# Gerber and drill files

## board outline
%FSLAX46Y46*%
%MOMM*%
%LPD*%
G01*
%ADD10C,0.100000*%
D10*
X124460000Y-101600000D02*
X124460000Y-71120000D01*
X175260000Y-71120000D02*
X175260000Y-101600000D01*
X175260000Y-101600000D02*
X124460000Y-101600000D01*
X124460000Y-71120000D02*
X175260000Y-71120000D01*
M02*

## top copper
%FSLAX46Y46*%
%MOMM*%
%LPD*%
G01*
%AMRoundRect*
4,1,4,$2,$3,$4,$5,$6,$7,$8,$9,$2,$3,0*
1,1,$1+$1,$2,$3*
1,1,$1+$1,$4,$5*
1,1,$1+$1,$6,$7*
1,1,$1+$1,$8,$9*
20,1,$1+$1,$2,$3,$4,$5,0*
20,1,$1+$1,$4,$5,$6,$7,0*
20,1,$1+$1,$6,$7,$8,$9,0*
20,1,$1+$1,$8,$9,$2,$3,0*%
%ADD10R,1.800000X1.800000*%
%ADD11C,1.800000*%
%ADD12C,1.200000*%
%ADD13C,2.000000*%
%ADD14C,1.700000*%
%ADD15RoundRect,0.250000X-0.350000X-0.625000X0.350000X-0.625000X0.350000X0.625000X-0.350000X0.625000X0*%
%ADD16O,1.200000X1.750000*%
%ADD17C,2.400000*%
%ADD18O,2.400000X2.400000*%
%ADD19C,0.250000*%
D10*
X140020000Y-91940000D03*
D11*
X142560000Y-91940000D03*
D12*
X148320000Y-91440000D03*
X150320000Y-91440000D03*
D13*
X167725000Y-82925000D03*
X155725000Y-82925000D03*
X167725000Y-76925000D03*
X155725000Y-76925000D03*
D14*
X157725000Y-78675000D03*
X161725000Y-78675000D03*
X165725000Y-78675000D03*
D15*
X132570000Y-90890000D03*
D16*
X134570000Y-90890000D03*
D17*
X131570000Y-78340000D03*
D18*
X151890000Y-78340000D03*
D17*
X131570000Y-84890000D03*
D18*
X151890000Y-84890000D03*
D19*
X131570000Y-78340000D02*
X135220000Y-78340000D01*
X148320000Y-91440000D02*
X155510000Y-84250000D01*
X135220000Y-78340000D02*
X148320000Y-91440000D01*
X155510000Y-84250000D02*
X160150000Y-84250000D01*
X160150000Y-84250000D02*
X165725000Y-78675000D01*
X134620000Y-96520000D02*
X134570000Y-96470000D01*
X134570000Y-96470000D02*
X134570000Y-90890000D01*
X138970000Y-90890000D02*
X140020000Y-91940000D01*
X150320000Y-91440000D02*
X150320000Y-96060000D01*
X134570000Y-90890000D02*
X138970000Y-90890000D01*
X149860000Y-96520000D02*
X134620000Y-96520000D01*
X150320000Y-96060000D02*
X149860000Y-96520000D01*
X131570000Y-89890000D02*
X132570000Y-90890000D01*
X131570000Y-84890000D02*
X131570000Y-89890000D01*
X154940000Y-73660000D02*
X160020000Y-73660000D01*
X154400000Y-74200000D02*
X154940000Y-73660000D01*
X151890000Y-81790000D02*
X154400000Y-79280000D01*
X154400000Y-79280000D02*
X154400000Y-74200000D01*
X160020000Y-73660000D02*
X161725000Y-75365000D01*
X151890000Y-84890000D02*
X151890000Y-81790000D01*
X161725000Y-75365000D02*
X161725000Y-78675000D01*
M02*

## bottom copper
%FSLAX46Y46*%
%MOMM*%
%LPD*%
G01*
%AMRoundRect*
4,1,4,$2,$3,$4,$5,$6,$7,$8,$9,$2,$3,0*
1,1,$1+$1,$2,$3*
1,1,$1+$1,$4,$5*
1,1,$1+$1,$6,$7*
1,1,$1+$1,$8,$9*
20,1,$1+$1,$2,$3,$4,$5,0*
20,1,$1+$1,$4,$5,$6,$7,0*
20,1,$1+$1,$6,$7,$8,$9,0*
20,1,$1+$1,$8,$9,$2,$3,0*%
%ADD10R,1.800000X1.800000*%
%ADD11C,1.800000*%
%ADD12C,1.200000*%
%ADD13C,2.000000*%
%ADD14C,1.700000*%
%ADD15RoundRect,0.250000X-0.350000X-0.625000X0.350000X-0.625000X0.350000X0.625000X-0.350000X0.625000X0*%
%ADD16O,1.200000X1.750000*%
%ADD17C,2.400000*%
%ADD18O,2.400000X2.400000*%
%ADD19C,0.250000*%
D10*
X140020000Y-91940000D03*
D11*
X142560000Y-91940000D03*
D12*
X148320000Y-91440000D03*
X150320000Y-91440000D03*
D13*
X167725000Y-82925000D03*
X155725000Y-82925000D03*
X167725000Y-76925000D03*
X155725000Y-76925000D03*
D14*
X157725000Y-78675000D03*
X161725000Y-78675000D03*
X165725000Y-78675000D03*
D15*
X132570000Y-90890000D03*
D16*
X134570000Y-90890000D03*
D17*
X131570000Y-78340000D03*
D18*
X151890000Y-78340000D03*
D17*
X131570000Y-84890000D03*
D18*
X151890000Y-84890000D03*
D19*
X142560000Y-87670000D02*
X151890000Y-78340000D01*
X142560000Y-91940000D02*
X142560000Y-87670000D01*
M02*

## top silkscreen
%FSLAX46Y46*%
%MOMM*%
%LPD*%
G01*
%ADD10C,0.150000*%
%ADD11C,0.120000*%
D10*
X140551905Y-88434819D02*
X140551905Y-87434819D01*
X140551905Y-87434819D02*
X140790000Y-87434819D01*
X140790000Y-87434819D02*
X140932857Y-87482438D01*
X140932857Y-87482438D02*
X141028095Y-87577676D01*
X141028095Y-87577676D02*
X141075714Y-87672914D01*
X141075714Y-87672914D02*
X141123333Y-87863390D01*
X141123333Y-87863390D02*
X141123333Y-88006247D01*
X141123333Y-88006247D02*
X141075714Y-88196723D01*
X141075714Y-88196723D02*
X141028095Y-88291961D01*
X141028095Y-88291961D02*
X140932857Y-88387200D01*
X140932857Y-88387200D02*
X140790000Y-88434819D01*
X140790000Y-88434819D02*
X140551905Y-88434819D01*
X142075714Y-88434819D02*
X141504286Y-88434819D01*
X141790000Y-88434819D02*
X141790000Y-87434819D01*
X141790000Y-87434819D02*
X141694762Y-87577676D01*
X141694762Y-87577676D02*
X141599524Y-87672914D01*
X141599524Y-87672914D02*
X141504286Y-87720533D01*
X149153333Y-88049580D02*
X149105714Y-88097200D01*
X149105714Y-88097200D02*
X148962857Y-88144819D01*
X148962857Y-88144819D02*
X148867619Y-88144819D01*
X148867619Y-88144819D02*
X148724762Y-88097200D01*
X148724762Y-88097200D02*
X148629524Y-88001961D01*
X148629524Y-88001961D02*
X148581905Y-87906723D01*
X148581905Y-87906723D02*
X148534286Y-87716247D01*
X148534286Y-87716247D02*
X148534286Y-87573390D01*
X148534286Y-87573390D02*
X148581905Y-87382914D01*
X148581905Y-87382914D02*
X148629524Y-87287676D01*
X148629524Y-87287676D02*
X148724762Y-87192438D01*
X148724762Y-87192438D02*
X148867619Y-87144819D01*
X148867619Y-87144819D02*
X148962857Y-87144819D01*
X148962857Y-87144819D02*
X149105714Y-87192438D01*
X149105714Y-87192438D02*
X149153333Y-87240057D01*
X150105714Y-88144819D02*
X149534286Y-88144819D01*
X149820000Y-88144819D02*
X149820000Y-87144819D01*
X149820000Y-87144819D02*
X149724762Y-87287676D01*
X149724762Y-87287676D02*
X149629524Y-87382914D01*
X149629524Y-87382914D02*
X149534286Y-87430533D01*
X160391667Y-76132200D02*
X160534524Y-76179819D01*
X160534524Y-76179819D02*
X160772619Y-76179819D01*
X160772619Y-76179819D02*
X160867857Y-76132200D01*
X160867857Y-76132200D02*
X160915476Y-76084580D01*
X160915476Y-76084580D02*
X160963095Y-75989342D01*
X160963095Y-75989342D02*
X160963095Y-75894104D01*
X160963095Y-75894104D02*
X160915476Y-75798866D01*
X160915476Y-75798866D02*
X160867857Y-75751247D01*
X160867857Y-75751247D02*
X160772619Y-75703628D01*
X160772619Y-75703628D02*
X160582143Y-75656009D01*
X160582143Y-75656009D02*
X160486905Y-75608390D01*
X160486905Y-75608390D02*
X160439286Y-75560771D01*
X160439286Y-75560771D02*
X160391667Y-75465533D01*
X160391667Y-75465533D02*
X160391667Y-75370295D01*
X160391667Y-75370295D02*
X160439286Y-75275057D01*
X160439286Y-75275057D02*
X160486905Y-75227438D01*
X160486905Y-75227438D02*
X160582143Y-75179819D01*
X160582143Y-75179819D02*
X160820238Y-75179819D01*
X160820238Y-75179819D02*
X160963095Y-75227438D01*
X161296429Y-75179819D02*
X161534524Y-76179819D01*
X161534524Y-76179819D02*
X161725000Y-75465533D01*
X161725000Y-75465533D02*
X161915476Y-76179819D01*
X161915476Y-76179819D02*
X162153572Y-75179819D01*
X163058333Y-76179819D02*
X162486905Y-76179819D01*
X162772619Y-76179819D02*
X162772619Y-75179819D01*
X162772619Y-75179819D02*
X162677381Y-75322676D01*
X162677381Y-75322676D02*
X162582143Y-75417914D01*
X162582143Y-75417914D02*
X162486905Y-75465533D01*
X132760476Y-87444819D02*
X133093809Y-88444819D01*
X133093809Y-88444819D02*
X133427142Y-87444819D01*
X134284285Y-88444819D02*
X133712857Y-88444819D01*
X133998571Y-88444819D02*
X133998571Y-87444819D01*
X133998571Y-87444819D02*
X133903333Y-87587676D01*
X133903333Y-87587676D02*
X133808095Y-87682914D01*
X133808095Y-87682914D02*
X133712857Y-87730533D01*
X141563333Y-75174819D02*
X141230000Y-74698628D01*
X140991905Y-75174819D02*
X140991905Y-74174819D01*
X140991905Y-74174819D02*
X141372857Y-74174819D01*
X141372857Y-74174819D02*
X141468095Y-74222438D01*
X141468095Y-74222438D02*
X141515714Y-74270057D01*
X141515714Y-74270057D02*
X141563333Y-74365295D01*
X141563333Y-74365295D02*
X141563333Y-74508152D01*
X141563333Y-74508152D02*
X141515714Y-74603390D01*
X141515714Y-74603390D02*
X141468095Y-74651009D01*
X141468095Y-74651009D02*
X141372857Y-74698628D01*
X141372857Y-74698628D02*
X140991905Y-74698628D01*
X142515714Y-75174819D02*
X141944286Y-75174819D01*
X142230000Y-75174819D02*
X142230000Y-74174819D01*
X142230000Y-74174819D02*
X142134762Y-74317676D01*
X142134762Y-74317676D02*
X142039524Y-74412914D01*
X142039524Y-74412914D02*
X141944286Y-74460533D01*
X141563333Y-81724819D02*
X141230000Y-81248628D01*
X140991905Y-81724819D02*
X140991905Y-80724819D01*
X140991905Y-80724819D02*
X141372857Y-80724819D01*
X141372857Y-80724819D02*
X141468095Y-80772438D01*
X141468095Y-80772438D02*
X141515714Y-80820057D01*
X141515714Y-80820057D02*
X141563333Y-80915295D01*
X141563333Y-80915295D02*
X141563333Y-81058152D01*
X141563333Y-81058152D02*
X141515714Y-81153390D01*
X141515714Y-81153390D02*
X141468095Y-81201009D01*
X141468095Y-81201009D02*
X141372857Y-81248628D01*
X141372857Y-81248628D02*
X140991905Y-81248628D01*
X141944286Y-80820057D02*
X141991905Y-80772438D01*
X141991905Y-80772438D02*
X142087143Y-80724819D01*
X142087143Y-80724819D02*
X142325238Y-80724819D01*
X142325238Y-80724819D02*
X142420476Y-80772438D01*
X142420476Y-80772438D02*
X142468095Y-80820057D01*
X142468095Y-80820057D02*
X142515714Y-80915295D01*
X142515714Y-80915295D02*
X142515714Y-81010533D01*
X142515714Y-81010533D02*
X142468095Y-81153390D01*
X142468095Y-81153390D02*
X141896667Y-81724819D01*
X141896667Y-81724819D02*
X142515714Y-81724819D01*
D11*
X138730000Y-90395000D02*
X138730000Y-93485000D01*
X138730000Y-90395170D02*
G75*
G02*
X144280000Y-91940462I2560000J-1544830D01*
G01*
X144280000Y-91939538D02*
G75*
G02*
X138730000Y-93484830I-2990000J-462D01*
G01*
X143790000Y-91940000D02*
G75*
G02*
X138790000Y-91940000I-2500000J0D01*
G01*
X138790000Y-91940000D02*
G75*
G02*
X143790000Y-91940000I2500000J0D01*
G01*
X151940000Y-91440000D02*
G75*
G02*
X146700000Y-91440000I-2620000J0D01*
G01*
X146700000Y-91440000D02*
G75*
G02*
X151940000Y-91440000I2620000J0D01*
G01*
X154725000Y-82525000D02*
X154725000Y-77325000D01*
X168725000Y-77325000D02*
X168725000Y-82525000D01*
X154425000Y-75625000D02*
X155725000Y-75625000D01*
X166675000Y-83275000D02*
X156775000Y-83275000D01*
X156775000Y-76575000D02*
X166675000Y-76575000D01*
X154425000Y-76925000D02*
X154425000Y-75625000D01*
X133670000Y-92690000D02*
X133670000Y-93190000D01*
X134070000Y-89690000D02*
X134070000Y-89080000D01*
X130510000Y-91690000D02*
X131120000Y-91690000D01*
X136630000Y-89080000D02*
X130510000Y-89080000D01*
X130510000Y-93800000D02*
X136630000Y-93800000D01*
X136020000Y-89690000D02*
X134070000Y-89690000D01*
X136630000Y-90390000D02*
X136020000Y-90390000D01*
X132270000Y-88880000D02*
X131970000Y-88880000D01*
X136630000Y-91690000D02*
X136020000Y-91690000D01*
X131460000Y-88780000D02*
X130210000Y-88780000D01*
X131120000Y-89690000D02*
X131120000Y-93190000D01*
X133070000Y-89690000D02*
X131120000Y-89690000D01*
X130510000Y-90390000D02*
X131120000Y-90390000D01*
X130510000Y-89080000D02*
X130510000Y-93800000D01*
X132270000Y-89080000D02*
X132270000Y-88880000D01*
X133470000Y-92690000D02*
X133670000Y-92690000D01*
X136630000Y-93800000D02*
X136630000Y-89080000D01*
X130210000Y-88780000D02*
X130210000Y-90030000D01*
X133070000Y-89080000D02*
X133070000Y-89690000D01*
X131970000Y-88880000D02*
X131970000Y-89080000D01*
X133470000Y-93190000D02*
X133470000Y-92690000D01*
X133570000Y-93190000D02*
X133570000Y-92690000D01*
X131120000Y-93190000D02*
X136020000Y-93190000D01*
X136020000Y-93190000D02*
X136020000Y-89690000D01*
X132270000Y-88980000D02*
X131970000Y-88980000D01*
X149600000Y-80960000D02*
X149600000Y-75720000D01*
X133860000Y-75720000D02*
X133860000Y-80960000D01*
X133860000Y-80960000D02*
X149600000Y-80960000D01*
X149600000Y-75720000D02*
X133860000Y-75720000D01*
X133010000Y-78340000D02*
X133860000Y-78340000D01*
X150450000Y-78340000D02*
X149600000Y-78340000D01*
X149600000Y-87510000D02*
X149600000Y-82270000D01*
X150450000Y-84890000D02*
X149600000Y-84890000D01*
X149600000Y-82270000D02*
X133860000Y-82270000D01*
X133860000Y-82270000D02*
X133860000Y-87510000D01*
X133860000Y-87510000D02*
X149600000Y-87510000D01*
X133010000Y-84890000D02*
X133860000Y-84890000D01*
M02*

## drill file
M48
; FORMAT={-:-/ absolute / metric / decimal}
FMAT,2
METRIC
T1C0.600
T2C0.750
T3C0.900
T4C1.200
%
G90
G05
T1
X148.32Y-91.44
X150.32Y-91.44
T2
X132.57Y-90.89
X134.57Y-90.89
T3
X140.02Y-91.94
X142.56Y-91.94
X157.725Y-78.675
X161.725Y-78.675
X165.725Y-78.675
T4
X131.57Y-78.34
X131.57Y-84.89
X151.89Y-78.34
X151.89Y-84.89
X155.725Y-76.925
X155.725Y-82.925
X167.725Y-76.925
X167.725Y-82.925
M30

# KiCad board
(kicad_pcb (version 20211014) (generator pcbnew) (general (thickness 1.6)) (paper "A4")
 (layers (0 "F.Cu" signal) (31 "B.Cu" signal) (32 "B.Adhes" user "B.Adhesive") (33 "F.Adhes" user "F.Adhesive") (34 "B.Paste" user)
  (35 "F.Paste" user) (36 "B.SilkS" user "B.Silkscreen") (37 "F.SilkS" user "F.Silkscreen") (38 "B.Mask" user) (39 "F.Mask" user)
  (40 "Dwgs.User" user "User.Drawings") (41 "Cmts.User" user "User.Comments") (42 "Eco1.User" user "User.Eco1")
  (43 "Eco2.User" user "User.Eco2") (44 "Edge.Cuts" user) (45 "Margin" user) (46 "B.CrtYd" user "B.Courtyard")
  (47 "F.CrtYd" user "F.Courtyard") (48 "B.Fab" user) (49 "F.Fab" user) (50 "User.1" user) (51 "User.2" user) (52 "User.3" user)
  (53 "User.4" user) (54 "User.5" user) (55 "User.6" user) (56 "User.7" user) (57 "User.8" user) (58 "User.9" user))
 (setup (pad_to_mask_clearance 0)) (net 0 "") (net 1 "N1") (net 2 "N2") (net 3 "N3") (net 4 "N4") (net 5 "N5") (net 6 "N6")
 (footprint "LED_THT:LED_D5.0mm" (layer "F.Cu") (at 140.02 91.94)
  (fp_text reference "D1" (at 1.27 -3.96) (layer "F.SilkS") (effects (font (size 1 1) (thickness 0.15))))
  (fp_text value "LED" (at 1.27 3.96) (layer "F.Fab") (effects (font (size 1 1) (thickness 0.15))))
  (fp_line (start -1.29 -1.545) (end -1.29 1.545) (layer "F.SilkS") (width 0.12))
  (fp_arc (start -1.29 -1.54483) (mid 2.072002 -2.880433) (end 4.26 0.000462) (layer "F.SilkS") (width 0.12))
  (fp_arc (start 4.26 -0.000462) (mid 2.072002 2.880433) (end -1.29 1.54483) (layer "F.SilkS") (width 0.12))
  (fp_circle (center 1.27 0) (end 3.77 0) (layer "F.SilkS") (width 0.12) (fill none))
  (pad "1" thru_hole rect (at 0 0) (size 1.8 1.8) (drill 0.9) (layers *.Cu *.Mask) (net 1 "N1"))
  (pad "2" thru_hole circle (at 2.54 0) (size 1.8 1.8) (drill 0.9) (layers *.Cu *.Mask) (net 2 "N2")))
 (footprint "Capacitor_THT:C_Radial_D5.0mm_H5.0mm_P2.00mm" (layer "F.Cu") (at 148.32 91.44)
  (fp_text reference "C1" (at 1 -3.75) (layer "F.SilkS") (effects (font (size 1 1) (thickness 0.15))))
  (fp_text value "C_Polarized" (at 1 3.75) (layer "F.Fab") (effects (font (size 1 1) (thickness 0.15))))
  (fp_circle (center 1 0) (end 3.62 0) (layer "F.SilkS") (width 0.12) (fill none))
  (pad "1" thru_hole circle (at 0 0) (size 1.2 1.2) (drill 0.6) (layers *.Cu *.Mask) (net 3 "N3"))
  (pad "2" thru_hole circle (at 2 0) (size 1.2 1.2) (drill 0.6) (layers *.Cu *.Mask) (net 1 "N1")))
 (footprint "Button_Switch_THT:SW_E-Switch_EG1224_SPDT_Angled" (layer "F.Cu") (at 157.725 78.675)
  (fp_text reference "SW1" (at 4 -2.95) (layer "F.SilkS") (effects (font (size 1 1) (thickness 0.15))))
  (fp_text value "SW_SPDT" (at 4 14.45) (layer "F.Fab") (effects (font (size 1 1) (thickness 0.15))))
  (fp_line (start -3 3.85) (end -3 -1.35) (layer "F.SilkS") (width 0.12))
  (fp_line (start 11 -1.35) (end 11 3.85) (layer "F.SilkS") (width 0.12))
  (fp_line (start -3.3 -3.05) (end -2 -3.05) (layer "F.SilkS") (width 0.12))
  (fp_line (start 8.95 4.6) (end -0.95 4.6) (layer "F.SilkS") (width 0.12))
  (fp_line (start -0.95 -2.1) (end 8.95 -2.1) (layer "F.SilkS") (width 0.12))
  (fp_line (start -3.3 -1.75) (end -3.3 -3.05) (layer "F.SilkS") (width 0.12))
  (pad "" thru_hole circle (at 10 4.25) (size 2 2) (drill 1.2) (layers *.Cu *.Mask))
  (pad "" thru_hole circle (at -2 4.25) (size 2 2) (drill 1.2) (layers *.Cu *.Mask))
  (pad "" thru_hole circle (at 10 -1.75) (size 2 2) (drill 1.2) (layers *.Cu *.Mask))
  (pad "" thru_hole circle (at -2 -1.75) (size 2 2) (drill 1.2) (layers *.Cu *.Mask))
  (pad "1" thru_hole circle (at 0 0) (size 1.7 1.7) (drill 0.9) (layers *.Cu *.Mask) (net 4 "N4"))
  (pad "2" thru_hole circle (at 4 0) (size 1.7 1.7) (drill 0.9) (layers *.Cu *.Mask) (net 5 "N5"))
  (pad "3" thru_hole circle (at 8 0) (size 1.7 1.7) (drill 0.9) (layers *.Cu *.Mask) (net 3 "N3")))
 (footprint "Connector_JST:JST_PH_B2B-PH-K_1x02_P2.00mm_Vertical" (layer "F.Cu") (at 132.57 90.89)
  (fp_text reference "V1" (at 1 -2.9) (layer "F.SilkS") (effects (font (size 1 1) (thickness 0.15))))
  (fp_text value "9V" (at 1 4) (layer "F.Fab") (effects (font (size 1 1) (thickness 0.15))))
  (fp_line (start 1.1 1.8) (end 1.1 2.3) (layer "F.SilkS") (width 0.12))
  (fp_line (start 1.5 -1.2) (end 1.5 -1.81) (layer "F.SilkS") (width 0.12))
  (fp_line (start -2.06 0.8) (end -1.45 0.8) (layer "F.SilkS") (width 0.12))
  (fp_line (start 4.06 -1.81) (end -2.06 -1.81) (layer "F.SilkS") (width 0.12))
  (fp_line (start -2.06 2.91) (end 4.06 2.91) (layer "F.SilkS") (width 0.12))
  (fp_line (start 3.45 -1.2) (end 1.5 -1.2) (layer "F.SilkS") (width 0.12))
  (fp_line (start 4.06 -0.5) (end 3.45 -0.5) (layer "F.SilkS") (width 0.12))
  (fp_line (start -0.3 -2.01) (end -0.6 -2.01) (layer "F.SilkS") (width 0.12))
  (fp_line (start 4.06 0.8) (end 3.45 0.8) (layer "F.SilkS") (width 0.12))
  (fp_line (start -1.11 -2.11) (end -2.36 -2.11) (layer "F.SilkS") (width 0.12))
  (fp_line (start -1.45 -1.2) (end -1.45 2.3) (layer "F.SilkS") (width 0.12))
  (fp_line (start 0.5 -1.2) (end -1.45 -1.2) (layer "F.SilkS") (width 0.12))
  (fp_line (start -2.06 -0.5) (end -1.45 -0.5) (layer "F.SilkS") (width 0.12))
  (fp_line (start -2.06 -1.81) (end -2.06 2.91) (layer "F.SilkS") (width 0.12))
  (fp_line (start -0.3 -1.81) (end -0.3 -2.01) (layer "F.SilkS") (width 0.12))
  (fp_line (start 0.9 1.8) (end 1.1 1.8) (layer "F.SilkS") (width 0.12))
  (fp_line (start 4.06 2.91) (end 4.06 -1.81) (layer "F.SilkS") (width 0.12))
  (fp_line (start -2.36 -2.11) (end -2.36 -0.86) (layer "F.SilkS") (width 0.12))
  (fp_line (start 0.5 -1.81) (end 0.5 -1.2) (layer "F.SilkS") (width 0.12))
  (fp_line (start -0.6 -2.01) (end -0.6 -1.81) (layer "F.SilkS") (width 0.12))
  (fp_line (start 0.9 2.3) (end 0.9 1.8) (layer "F.SilkS") (width 0.12))
  (fp_line (start 1 2.3) (end 1 1.8) (layer "F.SilkS") (width 0.12))
  (fp_line (start -1.45 2.3) (end 3.45 2.3) (layer "F.SilkS") (width 0.12))
  (fp_line (start 3.45 2.3) (end 3.45 -1.2) (layer "F.SilkS") (width 0.12))
  (fp_line (start -0.3 -1.91) (end -0.6 -1.91) (layer "F.SilkS") (width 0.12))
  (pad "1" thru_hole roundrect (at 0 0) (size 1.2 1.75) (drill 0.75) (layers *.Cu *.Mask) (roundrect_rratio 0.208333) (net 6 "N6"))
  (pad "2" thru_hole oval (at 2 0) (size 1.2 1.75) (drill 0.75) (layers *.Cu *.Mask) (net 1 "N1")))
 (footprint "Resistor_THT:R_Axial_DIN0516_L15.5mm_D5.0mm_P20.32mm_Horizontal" (layer "F.Cu") (at 131.57 78.34)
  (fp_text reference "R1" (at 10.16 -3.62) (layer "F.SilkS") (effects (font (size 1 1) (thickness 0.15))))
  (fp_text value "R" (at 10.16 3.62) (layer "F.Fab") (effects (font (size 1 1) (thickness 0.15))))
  (fp_line (start 18.03 2.62) (end 18.03 -2.62) (layer "F.SilkS") (width 0.12))
  (fp_line (start 2.29 -2.62) (end 2.29 2.62) (layer "F.SilkS") (width 0.12))
  (fp_line (start 2.29 2.62) (end 18.03 2.62) (layer "F.SilkS") (width 0.12))
  (fp_line (start 18.03 -2.62) (end 2.29 -2.62) (layer "F.SilkS") (width 0.12))
  (fp_line (start 1.44 0) (end 2.29 0) (layer "F.SilkS") (width 0.12))
  (fp_line (start 18.88 0) (end 18.03 0) (layer "F.SilkS") (width 0.12))
  (pad "1" thru_hole circle (at 0 0) (size 2.4 2.4) (drill 1.2) (layers *.Cu *.Mask) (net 3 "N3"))
  (pad "2" thru_hole oval (at 20.32 0) (size 2.4 2.4) (drill 1.2) (layers *.Cu *.Mask) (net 2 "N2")))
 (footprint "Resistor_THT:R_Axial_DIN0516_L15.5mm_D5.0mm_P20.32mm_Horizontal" (layer "F.Cu") (at 131.57 84.89)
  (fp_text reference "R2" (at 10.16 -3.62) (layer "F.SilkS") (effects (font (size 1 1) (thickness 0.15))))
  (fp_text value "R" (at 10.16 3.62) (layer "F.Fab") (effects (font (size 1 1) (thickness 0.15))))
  (fp_line (start 18.03 2.62) (end 18.03 -2.62) (layer "F.SilkS") (width 0.12))
  (fp_line (start 18.88 0) (end 18.03 0) (layer "F.SilkS") (width 0.12))
  (fp_line (start 18.03 -2.62) (end 2.29 -2.62) (layer "F.SilkS") (width 0.12))
  (fp_line (start 2.29 -2.62) (end 2.29 2.62) (layer "F.SilkS") (width 0.12))
  (fp_line (start 2.29 2.62) (end 18.03 2.62) (layer "F.SilkS") (width 0.12))
  (fp_line (start 1.44 0) (end 2.29 0) (layer "F.SilkS") (width 0.12))
  (pad "1" thru_hole circle (at 0 0) (size 2.4 2.4) (drill 1.2) (layers *.Cu *.Mask) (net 6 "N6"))
  (pad "2" thru_hole oval (at 20.32 0) (size 2.4 2.4) (drill 1.2) (layers *.Cu *.Mask) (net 5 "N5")))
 (gr_line (start 124.46 101.6) (end 124.46 71.12) (layer "Edge.Cuts") (width 0.1))
 (gr_line (start 175.26 71.12) (end 175.26 101.6) (layer "Edge.Cuts") (width 0.1))
 (gr_line (start 175.26 101.6) (end 124.46 101.6) (layer "Edge.Cuts") (width 0.1))
 (gr_line (start 124.46 71.12) (end 175.26 71.12) (layer "Edge.Cuts") (width 0.1))
 (segment (start 131.57 78.34) (end 135.22 78.34) (width 0.25) (layer "F.Cu") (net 3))
 (segment (start 148.32 91.44) (end 155.51 84.25) (width 0.25) (layer "F.Cu") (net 3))
 (segment (start 135.22 78.34) (end 148.32 91.44) (width 0.25) (layer "F.Cu") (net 3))
 (segment (start 155.51 84.25) (end 160.15 84.25) (width 0.25) (layer "F.Cu") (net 3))
 (segment (start 160.15 84.25) (end 165.725 78.675) (width 0.25) (layer "F.Cu") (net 3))
 (segment (start 134.62 96.52) (end 134.57 96.47) (width 0.25) (layer "F.Cu") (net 1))
 (segment (start 134.57 96.47) (end 134.57 90.89) (width 0.25) (layer "F.Cu") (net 1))
 (segment (start 138.97 90.89) (end 140.02 91.94) (width 0.25) (layer "F.Cu") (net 1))
 (segment (start 150.32 91.44) (end 150.32 96.06) (width 0.25) (layer "F.Cu") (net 1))
 (segment (start 134.57 90.89) (end 138.97 90.89) (width 0.25) (layer "F.Cu") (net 1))
 (segment (start 149.86 96.52) (end 134.62 96.52) (width 0.25) (layer "F.Cu") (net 1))
 (segment (start 150.32 96.06) (end 149.86 96.52) (width 0.25) (layer "F.Cu") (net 1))
 (segment (start 142.56 87.67) (end 151.89 78.34) (width 0.25) (layer "B.Cu") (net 2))
 (segment (start 142.56 91.94) (end 142.56 87.67) (width 0.25) (layer "B.Cu") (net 2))
 (segment (start 131.57 89.89) (end 132.57 90.89) (width 0.25) (layer "F.Cu") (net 6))
 (segment (start 131.57 84.89) (end 131.57 89.89) (width 0.25) (layer "F.Cu") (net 6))
 (segment (start 154.94 73.66) (end 160.02 73.66) (width 0.25) (layer "F.Cu") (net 5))
 (segment (start 154.4 74.2) (end 154.94 73.66) (width 0.25) (layer "F.Cu") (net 5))
 (segment (start 151.89 81.79) (end 154.4 79.28) (width 0.25) (layer "F.Cu") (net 5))
 (segment (start 154.4 79.28) (end 154.4 74.2) (width 0.25) (layer "F.Cu") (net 5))
 (segment (start 160.02 73.66) (end 161.725 75.365) (width 0.25) (layer "F.Cu") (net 5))
 (segment (start 151.89 84.89) (end 151.89 81.79) (width 0.25) (layer "F.Cu") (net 5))
 (segment (start 161.725 75.365) (end 161.725 78.675) (width 0.25) (layer "F.Cu") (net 5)))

